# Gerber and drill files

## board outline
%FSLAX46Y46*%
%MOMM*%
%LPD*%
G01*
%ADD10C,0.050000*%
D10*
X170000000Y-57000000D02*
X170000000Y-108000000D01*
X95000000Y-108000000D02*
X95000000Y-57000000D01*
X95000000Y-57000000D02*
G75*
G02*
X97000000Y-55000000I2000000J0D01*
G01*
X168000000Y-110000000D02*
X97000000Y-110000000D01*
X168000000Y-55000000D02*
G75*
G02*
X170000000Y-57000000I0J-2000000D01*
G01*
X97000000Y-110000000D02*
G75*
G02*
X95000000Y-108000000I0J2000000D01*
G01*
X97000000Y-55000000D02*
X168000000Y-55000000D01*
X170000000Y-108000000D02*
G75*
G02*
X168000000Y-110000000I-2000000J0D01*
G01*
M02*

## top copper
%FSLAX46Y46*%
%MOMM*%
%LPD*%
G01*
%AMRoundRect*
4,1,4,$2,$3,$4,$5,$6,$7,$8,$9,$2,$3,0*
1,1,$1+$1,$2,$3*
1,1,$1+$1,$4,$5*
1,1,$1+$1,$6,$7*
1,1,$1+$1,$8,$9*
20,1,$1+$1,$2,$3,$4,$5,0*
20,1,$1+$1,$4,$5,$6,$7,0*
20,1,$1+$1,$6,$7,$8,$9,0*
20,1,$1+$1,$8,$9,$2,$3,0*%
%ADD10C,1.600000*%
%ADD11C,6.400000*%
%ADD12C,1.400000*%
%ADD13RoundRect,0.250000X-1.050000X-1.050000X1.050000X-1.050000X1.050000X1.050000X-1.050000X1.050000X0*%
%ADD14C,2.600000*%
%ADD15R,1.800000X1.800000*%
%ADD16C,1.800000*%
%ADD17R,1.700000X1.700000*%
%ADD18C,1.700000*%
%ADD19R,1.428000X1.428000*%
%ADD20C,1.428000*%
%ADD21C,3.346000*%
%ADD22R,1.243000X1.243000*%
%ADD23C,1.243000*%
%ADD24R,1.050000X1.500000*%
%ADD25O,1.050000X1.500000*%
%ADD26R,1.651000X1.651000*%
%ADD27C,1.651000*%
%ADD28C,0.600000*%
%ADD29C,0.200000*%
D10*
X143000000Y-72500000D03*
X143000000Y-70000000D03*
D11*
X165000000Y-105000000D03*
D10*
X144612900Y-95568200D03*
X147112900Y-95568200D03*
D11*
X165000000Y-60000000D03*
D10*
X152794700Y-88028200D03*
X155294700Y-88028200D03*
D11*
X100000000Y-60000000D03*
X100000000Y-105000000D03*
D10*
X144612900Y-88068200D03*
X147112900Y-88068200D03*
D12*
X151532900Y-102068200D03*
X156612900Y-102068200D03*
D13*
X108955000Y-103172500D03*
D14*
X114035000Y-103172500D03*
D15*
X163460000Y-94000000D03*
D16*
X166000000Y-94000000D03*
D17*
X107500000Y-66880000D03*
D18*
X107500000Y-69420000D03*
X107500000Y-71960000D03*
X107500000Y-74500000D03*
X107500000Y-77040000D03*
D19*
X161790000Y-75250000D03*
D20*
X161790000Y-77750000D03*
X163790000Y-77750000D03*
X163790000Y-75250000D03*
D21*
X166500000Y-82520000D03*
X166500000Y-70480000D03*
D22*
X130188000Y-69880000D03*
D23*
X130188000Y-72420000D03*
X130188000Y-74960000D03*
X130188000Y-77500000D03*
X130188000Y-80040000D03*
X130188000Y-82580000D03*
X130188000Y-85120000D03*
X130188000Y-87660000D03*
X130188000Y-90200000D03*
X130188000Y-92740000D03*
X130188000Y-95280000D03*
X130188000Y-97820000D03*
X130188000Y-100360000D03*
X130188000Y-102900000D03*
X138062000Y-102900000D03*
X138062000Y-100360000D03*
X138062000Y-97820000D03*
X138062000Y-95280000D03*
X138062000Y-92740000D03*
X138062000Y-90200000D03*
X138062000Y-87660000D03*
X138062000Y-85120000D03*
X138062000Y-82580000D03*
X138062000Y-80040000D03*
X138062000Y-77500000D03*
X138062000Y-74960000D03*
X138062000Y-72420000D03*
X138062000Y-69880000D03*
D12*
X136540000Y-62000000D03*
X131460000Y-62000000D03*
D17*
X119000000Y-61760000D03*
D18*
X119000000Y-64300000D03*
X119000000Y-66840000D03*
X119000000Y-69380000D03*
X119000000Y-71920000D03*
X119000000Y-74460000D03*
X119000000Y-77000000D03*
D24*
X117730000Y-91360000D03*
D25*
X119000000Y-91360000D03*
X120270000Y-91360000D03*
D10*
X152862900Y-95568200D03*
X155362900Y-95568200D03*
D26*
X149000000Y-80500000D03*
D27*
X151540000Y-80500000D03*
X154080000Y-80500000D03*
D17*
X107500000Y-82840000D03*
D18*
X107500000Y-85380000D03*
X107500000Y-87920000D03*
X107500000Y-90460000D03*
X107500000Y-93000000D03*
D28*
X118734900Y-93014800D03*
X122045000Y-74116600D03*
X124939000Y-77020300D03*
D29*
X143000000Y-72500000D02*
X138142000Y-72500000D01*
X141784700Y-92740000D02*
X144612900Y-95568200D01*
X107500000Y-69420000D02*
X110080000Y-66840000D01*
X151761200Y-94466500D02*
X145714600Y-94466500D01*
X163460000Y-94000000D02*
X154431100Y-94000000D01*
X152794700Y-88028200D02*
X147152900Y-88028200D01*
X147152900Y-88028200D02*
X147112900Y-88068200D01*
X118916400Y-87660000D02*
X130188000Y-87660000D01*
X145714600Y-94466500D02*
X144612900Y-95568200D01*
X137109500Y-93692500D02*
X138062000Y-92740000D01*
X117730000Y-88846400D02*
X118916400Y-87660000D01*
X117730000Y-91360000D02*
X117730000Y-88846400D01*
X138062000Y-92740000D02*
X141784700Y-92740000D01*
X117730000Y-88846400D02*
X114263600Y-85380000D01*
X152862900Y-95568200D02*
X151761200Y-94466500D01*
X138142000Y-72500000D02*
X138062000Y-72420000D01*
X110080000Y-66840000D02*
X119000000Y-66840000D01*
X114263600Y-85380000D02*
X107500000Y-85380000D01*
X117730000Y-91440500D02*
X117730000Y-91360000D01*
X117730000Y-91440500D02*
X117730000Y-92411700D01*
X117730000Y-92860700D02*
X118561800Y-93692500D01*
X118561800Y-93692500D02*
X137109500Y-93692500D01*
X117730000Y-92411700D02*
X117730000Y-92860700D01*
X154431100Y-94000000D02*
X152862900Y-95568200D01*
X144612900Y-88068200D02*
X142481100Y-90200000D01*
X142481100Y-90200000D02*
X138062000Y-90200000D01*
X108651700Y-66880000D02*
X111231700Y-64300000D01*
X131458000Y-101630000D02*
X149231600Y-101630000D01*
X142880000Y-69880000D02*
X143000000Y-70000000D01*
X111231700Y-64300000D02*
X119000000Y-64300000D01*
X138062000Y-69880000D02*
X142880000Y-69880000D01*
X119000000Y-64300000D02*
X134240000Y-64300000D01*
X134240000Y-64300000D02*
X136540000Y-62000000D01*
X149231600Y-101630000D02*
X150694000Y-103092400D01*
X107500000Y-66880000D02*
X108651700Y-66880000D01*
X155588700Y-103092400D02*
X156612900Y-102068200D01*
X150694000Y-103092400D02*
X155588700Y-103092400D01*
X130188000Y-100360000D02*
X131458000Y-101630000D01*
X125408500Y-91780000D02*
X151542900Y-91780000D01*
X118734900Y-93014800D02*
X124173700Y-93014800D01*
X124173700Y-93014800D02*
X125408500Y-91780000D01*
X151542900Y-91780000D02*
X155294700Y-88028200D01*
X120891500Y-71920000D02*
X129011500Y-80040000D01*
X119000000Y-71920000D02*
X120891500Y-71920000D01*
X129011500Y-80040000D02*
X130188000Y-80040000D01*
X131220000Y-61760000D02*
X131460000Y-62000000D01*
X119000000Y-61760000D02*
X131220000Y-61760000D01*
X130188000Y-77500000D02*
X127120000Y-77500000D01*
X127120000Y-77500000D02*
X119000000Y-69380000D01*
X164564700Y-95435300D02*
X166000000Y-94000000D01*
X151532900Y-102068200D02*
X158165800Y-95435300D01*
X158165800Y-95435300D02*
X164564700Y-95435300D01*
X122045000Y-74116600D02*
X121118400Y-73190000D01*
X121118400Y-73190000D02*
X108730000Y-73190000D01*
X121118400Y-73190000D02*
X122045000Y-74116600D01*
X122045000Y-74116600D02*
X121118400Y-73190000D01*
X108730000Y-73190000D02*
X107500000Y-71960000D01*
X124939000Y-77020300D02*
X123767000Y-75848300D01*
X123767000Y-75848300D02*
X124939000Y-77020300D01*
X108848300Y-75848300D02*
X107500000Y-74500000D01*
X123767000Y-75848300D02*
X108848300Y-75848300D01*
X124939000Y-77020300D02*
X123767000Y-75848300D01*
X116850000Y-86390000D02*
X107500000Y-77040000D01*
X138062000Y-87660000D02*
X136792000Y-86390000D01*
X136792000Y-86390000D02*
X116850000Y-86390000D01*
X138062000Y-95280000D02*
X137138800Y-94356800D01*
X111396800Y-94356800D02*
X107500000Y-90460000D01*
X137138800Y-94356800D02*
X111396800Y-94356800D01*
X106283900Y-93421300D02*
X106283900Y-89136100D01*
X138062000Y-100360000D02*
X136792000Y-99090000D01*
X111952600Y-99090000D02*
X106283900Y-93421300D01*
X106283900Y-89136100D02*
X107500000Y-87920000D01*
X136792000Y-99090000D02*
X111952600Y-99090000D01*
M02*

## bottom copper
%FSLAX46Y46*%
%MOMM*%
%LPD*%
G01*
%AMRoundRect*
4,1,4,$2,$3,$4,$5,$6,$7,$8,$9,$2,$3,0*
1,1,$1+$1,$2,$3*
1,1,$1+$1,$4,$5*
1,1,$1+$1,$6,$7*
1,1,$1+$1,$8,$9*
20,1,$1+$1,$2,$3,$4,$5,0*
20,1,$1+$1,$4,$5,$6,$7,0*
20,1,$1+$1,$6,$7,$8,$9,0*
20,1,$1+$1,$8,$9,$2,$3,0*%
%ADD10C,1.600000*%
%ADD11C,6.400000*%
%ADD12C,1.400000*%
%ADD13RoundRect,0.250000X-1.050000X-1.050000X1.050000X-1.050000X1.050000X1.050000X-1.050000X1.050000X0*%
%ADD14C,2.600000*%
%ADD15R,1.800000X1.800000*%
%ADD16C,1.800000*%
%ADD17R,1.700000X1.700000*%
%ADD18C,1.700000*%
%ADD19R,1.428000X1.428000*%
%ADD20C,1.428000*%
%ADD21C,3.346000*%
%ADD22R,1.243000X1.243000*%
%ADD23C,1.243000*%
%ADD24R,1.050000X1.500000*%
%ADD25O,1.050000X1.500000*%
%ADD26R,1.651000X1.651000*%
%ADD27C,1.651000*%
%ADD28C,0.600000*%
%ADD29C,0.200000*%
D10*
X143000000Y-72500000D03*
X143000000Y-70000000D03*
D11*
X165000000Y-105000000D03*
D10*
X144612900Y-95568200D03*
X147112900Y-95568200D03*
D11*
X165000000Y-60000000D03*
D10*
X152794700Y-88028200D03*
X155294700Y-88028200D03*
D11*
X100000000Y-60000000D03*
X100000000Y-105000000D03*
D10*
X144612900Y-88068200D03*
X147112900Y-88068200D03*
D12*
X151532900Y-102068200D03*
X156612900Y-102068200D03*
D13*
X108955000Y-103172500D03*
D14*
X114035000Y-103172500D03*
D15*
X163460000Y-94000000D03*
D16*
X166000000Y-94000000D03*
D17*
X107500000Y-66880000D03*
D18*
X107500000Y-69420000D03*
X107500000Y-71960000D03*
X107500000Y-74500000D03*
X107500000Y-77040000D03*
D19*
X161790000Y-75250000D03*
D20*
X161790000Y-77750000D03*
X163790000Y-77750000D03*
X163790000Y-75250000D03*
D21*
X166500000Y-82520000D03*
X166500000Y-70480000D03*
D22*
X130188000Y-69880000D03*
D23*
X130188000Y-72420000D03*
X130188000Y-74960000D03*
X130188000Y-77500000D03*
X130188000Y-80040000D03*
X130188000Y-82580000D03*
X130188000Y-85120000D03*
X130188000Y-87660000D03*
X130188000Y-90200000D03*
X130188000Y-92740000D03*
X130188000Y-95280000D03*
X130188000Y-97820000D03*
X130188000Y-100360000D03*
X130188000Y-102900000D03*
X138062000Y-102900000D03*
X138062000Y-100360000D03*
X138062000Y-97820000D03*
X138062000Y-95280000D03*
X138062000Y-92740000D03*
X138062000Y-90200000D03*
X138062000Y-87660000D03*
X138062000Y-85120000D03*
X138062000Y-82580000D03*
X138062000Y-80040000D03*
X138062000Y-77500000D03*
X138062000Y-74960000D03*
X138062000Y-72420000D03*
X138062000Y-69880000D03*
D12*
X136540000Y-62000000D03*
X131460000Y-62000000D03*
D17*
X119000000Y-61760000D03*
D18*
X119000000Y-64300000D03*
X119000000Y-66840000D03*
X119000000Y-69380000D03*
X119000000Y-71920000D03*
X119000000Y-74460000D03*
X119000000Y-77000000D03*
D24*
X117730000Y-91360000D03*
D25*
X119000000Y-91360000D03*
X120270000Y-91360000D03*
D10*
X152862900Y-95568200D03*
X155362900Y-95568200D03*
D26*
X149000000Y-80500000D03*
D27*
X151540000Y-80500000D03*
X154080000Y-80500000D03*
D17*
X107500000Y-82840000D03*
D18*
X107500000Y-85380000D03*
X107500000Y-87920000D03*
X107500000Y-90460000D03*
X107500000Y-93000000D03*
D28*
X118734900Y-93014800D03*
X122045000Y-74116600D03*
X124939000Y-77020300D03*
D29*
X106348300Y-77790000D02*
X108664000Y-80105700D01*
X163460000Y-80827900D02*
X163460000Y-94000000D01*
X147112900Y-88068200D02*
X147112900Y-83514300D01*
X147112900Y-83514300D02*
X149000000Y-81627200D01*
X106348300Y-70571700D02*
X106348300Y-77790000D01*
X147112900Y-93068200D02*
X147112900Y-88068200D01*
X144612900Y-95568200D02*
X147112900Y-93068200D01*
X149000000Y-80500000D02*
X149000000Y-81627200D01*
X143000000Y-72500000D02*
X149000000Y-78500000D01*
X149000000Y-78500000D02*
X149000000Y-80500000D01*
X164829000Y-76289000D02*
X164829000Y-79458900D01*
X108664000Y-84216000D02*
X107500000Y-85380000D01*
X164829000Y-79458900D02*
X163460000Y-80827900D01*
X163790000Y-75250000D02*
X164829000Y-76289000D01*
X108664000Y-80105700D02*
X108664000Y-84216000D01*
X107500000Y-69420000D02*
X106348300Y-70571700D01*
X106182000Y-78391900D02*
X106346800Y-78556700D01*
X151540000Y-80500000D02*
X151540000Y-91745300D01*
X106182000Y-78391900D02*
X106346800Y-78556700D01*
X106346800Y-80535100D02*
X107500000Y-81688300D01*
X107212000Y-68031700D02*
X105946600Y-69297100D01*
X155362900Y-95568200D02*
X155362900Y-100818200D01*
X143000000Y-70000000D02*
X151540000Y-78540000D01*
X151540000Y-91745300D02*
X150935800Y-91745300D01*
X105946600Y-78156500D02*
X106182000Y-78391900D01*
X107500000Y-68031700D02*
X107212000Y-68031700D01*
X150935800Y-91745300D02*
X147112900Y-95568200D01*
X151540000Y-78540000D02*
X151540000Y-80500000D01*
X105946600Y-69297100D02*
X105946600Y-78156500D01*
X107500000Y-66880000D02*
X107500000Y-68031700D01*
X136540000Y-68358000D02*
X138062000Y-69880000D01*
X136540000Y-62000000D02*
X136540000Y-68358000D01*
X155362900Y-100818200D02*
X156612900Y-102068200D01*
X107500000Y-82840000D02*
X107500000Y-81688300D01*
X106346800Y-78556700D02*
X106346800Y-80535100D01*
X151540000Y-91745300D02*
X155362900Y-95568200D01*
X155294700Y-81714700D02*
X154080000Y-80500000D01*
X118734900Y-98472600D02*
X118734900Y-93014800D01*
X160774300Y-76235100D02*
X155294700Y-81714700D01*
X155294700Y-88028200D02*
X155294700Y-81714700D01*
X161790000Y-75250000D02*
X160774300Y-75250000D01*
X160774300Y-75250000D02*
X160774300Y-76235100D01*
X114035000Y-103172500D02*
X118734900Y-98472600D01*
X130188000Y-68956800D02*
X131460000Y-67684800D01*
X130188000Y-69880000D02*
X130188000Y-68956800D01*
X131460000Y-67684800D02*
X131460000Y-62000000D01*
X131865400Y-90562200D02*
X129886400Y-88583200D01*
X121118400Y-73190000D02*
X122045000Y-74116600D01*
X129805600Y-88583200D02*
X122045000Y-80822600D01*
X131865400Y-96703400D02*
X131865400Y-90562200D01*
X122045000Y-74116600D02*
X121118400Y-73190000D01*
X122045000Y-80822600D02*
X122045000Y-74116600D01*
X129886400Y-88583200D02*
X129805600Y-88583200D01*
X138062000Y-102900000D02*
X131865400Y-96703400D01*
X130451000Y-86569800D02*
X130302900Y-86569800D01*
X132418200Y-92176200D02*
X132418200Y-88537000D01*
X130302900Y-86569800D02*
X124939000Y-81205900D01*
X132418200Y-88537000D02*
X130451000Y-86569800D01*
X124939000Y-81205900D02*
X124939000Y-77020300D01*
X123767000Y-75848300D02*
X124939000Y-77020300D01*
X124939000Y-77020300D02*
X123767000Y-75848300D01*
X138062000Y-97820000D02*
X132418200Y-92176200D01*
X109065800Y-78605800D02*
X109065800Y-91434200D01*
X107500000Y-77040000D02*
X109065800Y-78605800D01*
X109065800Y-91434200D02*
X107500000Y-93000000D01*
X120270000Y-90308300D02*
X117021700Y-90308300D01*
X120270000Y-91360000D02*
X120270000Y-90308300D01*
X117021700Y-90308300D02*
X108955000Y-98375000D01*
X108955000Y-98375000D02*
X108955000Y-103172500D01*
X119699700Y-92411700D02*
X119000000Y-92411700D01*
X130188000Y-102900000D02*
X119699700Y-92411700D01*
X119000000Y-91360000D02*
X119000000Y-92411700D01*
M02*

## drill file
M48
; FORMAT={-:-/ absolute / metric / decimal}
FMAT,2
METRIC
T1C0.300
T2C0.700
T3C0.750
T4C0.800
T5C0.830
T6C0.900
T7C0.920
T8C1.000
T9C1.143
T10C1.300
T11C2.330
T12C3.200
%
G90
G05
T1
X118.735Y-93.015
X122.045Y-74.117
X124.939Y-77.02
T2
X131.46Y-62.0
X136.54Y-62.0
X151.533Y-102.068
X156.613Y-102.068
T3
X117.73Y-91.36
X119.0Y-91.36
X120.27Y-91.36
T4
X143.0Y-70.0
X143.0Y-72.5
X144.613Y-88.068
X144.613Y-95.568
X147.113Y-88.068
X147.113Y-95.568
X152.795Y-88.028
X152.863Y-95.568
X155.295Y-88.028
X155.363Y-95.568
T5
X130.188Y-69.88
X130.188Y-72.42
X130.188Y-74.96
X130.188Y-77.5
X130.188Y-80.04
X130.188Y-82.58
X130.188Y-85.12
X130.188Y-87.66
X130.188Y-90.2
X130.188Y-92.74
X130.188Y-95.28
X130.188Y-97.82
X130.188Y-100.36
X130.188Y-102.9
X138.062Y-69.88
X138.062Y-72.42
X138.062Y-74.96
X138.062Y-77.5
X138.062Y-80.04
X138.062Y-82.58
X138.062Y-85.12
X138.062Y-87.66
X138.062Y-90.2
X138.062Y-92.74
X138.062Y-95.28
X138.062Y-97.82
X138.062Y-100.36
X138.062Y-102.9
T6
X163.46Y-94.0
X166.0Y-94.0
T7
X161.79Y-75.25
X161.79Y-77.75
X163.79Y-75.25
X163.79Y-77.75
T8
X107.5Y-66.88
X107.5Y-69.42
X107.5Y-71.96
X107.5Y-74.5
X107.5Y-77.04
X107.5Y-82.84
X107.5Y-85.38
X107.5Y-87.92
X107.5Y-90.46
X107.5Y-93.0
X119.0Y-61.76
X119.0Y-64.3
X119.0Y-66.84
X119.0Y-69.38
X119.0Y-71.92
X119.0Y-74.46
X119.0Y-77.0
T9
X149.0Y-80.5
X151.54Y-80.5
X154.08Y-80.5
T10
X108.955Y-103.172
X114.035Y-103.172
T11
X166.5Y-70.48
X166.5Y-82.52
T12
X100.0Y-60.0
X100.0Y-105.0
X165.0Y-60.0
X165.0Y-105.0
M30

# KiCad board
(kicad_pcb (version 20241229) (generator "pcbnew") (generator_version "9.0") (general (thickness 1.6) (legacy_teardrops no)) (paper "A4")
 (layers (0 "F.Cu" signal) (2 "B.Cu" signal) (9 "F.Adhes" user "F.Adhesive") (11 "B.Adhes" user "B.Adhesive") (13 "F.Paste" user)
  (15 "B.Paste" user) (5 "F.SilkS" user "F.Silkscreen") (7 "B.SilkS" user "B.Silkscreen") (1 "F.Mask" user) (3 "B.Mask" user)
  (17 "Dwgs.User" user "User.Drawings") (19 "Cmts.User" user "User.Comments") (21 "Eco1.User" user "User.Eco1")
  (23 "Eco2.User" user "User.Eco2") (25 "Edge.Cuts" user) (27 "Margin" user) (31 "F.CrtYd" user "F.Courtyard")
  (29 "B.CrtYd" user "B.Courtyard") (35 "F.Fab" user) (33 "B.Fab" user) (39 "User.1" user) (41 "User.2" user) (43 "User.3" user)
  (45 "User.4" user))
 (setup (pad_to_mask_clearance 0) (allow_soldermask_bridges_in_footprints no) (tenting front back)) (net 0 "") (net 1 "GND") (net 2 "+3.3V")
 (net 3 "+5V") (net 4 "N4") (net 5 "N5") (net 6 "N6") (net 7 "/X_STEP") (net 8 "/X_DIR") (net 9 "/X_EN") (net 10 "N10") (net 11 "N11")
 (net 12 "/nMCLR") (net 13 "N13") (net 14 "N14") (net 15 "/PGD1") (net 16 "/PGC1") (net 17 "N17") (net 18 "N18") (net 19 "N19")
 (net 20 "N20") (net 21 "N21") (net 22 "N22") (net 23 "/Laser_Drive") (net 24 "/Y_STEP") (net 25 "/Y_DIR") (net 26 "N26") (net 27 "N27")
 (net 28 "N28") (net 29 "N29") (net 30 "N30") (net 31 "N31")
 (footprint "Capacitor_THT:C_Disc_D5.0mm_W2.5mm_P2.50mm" (layer "F.Cu") (at 143 72.5 90)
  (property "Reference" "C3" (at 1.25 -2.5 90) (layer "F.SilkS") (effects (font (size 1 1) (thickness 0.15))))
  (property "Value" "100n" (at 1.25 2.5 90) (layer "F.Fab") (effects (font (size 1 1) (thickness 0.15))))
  (pad "1" thru_hole circle (at 0 0 90) (size 1.6 1.6) (drill 0.8) (layers "*.Cu" "*.Mask") (remove_unused_layers no) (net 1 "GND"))
  (pad "2" thru_hole circle (at 2.5 0 90) (size 1.6 1.6) (drill 0.8) (layers "*.Cu" "*.Mask") (remove_unused_layers no) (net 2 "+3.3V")))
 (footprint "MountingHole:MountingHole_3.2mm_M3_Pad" (layer "F.Cu") (at 165 105)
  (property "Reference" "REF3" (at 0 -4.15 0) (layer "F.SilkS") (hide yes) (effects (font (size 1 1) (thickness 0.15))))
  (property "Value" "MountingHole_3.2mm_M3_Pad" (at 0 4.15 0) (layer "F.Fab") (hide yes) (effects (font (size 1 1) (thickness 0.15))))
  (pad "1" thru_hole circle (at 0 0) (size 6.4 6.4) (drill 3.2) (layers "*.Cu" "*.Mask") (remove_unused_layers no) (zone_connect 2)))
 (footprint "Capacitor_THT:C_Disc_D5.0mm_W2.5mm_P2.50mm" (layer "F.Cu") (at 144.6129 95.5682)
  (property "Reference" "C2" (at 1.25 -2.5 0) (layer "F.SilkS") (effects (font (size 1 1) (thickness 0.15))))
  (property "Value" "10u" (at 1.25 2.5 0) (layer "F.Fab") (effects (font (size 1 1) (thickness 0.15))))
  (pad "1" thru_hole circle (at 0 0) (size 1.6 1.6) (drill 0.8) (layers "*.Cu" "*.Mask") (remove_unused_layers no) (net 1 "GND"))
  (pad "2" thru_hole circle (at 2.5 0) (size 1.6 1.6) (drill 0.8) (layers "*.Cu" "*.Mask") (remove_unused_layers no) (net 2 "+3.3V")))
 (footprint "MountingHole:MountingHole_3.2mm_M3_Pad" (layer "F.Cu") (at 165 60)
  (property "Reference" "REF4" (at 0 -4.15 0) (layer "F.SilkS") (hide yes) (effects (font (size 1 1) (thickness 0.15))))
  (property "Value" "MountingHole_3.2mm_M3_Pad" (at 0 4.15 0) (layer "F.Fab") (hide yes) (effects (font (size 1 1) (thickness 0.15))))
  (pad "1" thru_hole circle (at 0 0) (size 6.4 6.4) (drill 3.2) (layers "*.Cu" "*.Mask") (remove_unused_layers no) (zone_connect 2)))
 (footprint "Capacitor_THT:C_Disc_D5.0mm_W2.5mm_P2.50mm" (layer "F.Cu") (at 152.7947 88.0282)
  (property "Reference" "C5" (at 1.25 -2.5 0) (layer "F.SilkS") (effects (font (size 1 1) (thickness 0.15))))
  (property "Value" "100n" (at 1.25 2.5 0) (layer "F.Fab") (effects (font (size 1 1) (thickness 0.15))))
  (pad "1" thru_hole circle (at 0 0) (size 1.6 1.6) (drill 0.8) (layers "*.Cu" "*.Mask") (remove_unused_layers no) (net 1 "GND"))
  (pad "2" thru_hole circle (at 2.5 0) (size 1.6 1.6) (drill 0.8) (layers "*.Cu" "*.Mask") (remove_unused_layers no) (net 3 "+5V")))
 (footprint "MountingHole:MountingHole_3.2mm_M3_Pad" (layer "F.Cu") (at 100 60)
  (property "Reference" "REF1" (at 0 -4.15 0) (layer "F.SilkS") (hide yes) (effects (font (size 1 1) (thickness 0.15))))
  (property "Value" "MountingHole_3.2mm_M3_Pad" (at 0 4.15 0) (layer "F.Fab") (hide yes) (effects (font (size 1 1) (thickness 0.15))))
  (pad "1" thru_hole circle (at 0 0) (size 6.4 6.4) (drill 3.2) (layers "*.Cu" "*.Mask") (remove_unused_layers no) (zone_connect 2)))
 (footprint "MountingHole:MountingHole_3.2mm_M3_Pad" (layer "F.Cu") (at 100 105)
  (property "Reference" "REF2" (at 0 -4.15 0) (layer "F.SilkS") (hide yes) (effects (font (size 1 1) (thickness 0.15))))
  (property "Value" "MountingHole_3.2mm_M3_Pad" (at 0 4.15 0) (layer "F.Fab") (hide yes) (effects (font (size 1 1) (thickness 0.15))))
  (pad "1" thru_hole circle (at 0 0) (size 6.4 6.4) (drill 3.2) (layers "*.Cu" "*.Mask") (remove_unused_layers no) (zone_connect 2)))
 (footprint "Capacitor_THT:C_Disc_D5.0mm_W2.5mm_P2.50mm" (layer "F.Cu") (at 144.6129 88.0682)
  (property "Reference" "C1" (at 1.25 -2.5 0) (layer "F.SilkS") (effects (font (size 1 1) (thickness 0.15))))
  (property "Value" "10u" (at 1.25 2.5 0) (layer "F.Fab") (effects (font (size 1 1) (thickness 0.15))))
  (pad "1" thru_hole circle (at 0 0) (size 1.6 1.6) (drill 0.8) (layers "*.Cu" "*.Mask") (remove_unused_layers no) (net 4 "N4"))
  (pad "2" thru_hole circle (at 2.5 0) (size 1.6 1.6) (drill 0.8) (layers "*.Cu" "*.Mask") (remove_unused_layers no) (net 1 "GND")))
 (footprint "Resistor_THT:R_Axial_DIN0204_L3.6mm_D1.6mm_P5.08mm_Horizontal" (layer "F.Cu") (at 151.5329 102.0682)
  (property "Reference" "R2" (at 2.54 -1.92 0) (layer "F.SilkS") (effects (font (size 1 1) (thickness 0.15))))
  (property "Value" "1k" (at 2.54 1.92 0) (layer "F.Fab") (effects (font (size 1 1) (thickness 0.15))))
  (pad "1" thru_hole circle (at 0 0) (size 1.4 1.4) (drill 0.7) (layers "*.Cu" "*.Mask") (remove_unused_layers no) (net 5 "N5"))
  (pad "2" thru_hole circle (at 5.08 0) (size 1.4 1.4) (drill 0.7) (layers "*.Cu" "*.Mask") (remove_unused_layers no) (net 2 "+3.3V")))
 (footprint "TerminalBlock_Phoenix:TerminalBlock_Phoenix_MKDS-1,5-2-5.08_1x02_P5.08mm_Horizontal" (layer "F.Cu") (at 108.955 103.1725)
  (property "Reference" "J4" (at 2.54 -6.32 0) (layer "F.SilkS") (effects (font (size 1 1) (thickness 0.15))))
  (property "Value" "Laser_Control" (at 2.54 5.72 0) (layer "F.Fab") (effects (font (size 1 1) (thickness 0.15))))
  (pad "1" thru_hole roundrect (at 0 0) (size 2.6 2.6) (drill 1.3) (layers "*.Cu" "*.Mask") (remove_unused_layers no)
   (roundrect_rratio 0.096154) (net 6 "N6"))
  (pad "2" thru_hole circle (at 5.08 0) (size 2.6 2.6) (drill 1.3) (layers "*.Cu" "*.Mask") (remove_unused_layers no) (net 3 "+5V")))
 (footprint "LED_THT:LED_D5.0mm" (layer "F.Cu") (at 163.46 94)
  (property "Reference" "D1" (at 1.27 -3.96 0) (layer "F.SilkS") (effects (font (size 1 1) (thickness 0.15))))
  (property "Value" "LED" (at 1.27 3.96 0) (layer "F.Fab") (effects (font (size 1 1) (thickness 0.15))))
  (pad "1" thru_hole rect (at 0 0) (size 1.8 1.8) (drill 0.9) (layers "*.Cu" "*.Mask") (remove_unused_layers no) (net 1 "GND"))
  (pad "2" thru_hole circle (at 2.54 0) (size 1.8 1.8) (drill 0.9) (layers "*.Cu" "*.Mask") (remove_unused_layers no) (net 5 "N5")))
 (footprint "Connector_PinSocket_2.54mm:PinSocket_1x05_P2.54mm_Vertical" (layer "F.Cu") (at 107.5 66.88)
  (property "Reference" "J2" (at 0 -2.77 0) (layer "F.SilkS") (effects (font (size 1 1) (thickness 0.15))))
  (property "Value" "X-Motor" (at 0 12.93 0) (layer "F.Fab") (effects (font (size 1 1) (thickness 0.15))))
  (pad "1" thru_hole rect (at 0 0) (size 1.7 1.7) (drill 1) (layers "*.Cu" "*.Mask") (remove_unused_layers no) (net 2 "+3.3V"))
  (pad "2" thru_hole circle (at 0 2.54) (size 1.7 1.7) (drill 1) (layers "*.Cu" "*.Mask") (remove_unused_layers no) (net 1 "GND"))
  (pad "3" thru_hole circle (at 0 5.08) (size 1.7 1.7) (drill 1) (layers "*.Cu" "*.Mask") (remove_unused_layers no) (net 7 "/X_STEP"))
  (pad "4" thru_hole circle (at 0 7.62) (size 1.7 1.7) (drill 1) (layers "*.Cu" "*.Mask") (remove_unused_layers no) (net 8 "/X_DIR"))
  (pad "5" thru_hole circle (at 0 10.16) (size 1.7 1.7) (drill 1) (layers "*.Cu" "*.Mask") (remove_unused_layers no) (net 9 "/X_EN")))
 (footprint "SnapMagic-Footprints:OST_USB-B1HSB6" (layer "F.Cu") (at 166.5 76.5 90)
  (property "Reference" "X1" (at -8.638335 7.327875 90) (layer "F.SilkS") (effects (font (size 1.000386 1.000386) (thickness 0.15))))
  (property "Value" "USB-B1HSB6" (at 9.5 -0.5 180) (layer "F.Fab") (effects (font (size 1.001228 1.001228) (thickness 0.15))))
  (pad "1" thru_hole rect (at 1.25 -4.71 90) (size 1.428 1.428) (drill 0.92) (layers "*.Cu" "*.Mask") (remove_unused_layers no)
   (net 3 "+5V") (solder_mask_margin 0.102))
  (pad "2" thru_hole circle (at -1.25 -4.71 90) (size 1.428 1.428) (drill 0.92) (layers "*.Cu" "*.Mask") (remove_unused_layers no)
   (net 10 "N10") (solder_mask_margin 0.102))
  (pad "3" thru_hole circle (at -1.25 -2.71 90) (size 1.428 1.428) (drill 0.92) (layers "*.Cu" "*.Mask") (remove_unused_layers no)
   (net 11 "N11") (solder_mask_margin 0.102))
  (pad "4" thru_hole circle (at 1.25 -2.71 90) (size 1.428 1.428) (drill 0.92) (layers "*.Cu" "*.Mask") (remove_unused_layers no)
   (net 1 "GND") (solder_mask_margin 0.102))
  (pad "P1" thru_hole circle (at -6.02 0 90) (size 3.346 3.346) (drill 2.33) (layers "*.Cu" "*.Mask") (remove_unused_layers no)
   (solder_mask_margin 0.102))
  (pad "P2" thru_hole circle (at 6.02 0 90) (size 3.346 3.346) (drill 2.33) (layers "*.Cu" "*.Mask") (remove_unused_layers no)
   (solder_mask_margin 0.102)))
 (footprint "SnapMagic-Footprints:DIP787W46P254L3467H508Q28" (layer "F.Cu") (at 134.125 86.39)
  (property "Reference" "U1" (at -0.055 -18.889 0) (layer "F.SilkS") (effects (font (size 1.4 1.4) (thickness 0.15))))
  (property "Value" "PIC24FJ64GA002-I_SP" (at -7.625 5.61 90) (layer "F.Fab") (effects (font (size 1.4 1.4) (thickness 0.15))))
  (pad "1" thru_hole rect (at -3.937 -16.51) (size 1.243 1.243) (drill 0.83) (layers "*.Cu" "*.Mask") (remove_unused_layers no)
   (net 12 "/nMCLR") (solder_mask_margin 0.102))
  (pad "2" thru_hole circle (at -3.937 -13.97) (size 1.243 1.243) (drill 0.83) (layers "*.Cu" "*.Mask") (remove_unused_layers no)
   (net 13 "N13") (solder_mask_margin 0.102))
  (pad "3" thru_hole circle (at -3.937 -11.43) (size 1.243 1.243) (drill 0.83) (layers "*.Cu" "*.Mask") (remove_unused_layers no)
   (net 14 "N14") (solder_mask_margin 0.102))
  (pad "4" thru_hole circle (at -3.937 -8.89) (size 1.243 1.243) (drill 0.83) (layers "*.Cu" "*.Mask") (remove_unused_layers no)
   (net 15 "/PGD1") (solder_mask_margin 0.102))
  (pad "5" thru_hole circle (at -3.937 -6.35) (size 1.243 1.243) (drill 0.83) (layers "*.Cu" "*.Mask") (remove_unused_layers no)
   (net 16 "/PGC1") (solder_mask_margin 0.102))
  (pad "6" thru_hole circle (at -3.937 -3.81) (size 1.243 1.243) (drill 0.83) (layers "*.Cu" "*.Mask") (remove_unused_layers no)
   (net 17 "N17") (solder_mask_margin 0.102))
  (pad "7" thru_hole circle (at -3.937 -1.27) (size 1.243 1.243) (drill 0.83) (layers "*.Cu" "*.Mask") (remove_unused_layers no)
   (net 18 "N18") (solder_mask_margin 0.102))
  (pad "8" thru_hole circle (at -3.937 1.27) (size 1.243 1.243) (drill 0.83) (layers "*.Cu" "*.Mask") (remove_unused_layers no)
   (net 1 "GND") (solder_mask_margin 0.102))
  (pad "9" thru_hole circle (at -3.937 3.81) (size 1.243 1.243) (drill 0.83) (layers "*.Cu" "*.Mask") (remove_unused_layers no)
   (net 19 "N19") (solder_mask_margin 0.102))
  (pad "10" thru_hole circle (at -3.937 6.35) (size 1.243 1.243) (drill 0.83) (layers "*.Cu" "*.Mask") (remove_unused_layers no)
   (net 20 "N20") (solder_mask_margin 0.102))
  (pad "11" thru_hole circle (at -3.937 8.89) (size 1.243 1.243) (drill 0.83) (layers "*.Cu" "*.Mask") (remove_unused_layers no)
   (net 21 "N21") (solder_mask_margin 0.102))
  (pad "12" thru_hole circle (at -3.937 11.43) (size 1.243 1.243) (drill 0.83) (layers "*.Cu" "*.Mask") (remove_unused_layers no)
   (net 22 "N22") (solder_mask_margin 0.102))
  (pad "13" thru_hole circle (at -3.937 13.97) (size 1.243 1.243) (drill 0.83) (layers "*.Cu" "*.Mask") (remove_unused_layers no)
   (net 2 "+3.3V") (solder_mask_margin 0.102))
  (pad "14" thru_hole circle (at -3.937 16.51) (size 1.243 1.243) (drill 0.83) (layers "*.Cu" "*.Mask") (remove_unused_layers no)
   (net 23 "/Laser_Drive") (solder_mask_margin 0.102))
  (pad "15" thru_hole circle (at 3.937 16.51) (size 1.243 1.243) (drill 0.83) (layers "*.Cu" "*.Mask") (remove_unused_layers no)
   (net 7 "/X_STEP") (solder_mask_margin 0.102))
  (pad "16" thru_hole circle (at 3.937 13.97) (size 1.243 1.243) (drill 0.83) (layers "*.Cu" "*.Mask") (remove_unused_layers no)
   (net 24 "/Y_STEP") (solder_mask_margin 0.102))
  (pad "17" thru_hole circle (at 3.937 11.43) (size 1.243 1.243) (drill 0.83) (layers "*.Cu" "*.Mask") (remove_unused_layers no)
   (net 8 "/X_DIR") (solder_mask_margin 0.102))
  (pad "18" thru_hole circle (at 3.937 8.89) (size 1.243 1.243) (drill 0.83) (layers "*.Cu" "*.Mask") (remove_unused_layers no)
   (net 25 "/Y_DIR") (solder_mask_margin 0.102))
  (pad "19" thru_hole circle (at 3.937 6.35) (size 1.243 1.243) (drill 0.83) (layers "*.Cu" "*.Mask") (remove_unused_layers no)
   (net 1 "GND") (solder_mask_margin 0.102))
  (pad "20" thru_hole circle (at 3.937 3.81) (size 1.243 1.243) (drill 0.83) (layers "*.Cu" "*.Mask") (remove_unused_layers no) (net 4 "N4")
   (solder_mask_margin 0.102))
  (pad "21" thru_hole circle (at 3.937 1.27) (size 1.243 1.243) (drill 0.83) (layers "*.Cu" "*.Mask") (remove_unused_layers no)
   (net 9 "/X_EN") (solder_mask_margin 0.102))
  (pad "22" thru_hole circle (at 3.937 -1.27) (size 1.243 1.243) (drill 0.83) (layers "*.Cu" "*.Mask") (remove_unused_layers no)
   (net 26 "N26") (solder_mask_margin 0.102))
  (pad "23" thru_hole circle (at 3.937 -3.81) (size 1.243 1.243) (drill 0.83) (layers "*.Cu" "*.Mask") (remove_unused_layers no)
   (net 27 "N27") (solder_mask_margin 0.102))
  (pad "24" thru_hole circle (at 3.937 -6.35) (size 1.243 1.243) (drill 0.83) (layers "*.Cu" "*.Mask") (remove_unused_layers no)
   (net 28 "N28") (solder_mask_margin 0.102))
  (pad "25" thru_hole circle (at 3.937 -8.89) (size 1.243 1.243) (drill 0.83) (layers "*.Cu" "*.Mask") (remove_unused_layers no)
   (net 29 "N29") (solder_mask_margin 0.102))
  (pad "26" thru_hole circle (at 3.937 -11.43) (size 1.243 1.243) (drill 0.83) (layers "*.Cu" "*.Mask") (remove_unused_layers no)
   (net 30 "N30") (solder_mask_margin 0.102))
  (pad "27" thru_hole circle (at 3.937 -13.97) (size 1.243 1.243) (drill 0.83) (layers "*.Cu" "*.Mask") (remove_unused_layers no)
   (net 1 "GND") (solder_mask_margin 0.102))
  (pad "28" thru_hole circle (at 3.937 -16.51) (size 1.243 1.243) (drill 0.83) (layers "*.Cu" "*.Mask") (remove_unused_layers no)
   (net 2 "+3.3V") (solder_mask_margin 0.102)))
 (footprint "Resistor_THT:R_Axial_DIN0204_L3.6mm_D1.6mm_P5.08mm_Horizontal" (layer "F.Cu") (at 136.54 62 180)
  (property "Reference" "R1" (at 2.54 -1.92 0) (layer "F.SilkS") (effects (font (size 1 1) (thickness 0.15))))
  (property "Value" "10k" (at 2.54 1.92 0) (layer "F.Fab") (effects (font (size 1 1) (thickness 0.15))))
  (pad "1" thru_hole circle (at 0 0 180) (size 1.4 1.4) (drill 0.7) (layers "*.Cu" "*.Mask") (remove_unused_layers no) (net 2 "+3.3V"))
  (pad "2" thru_hole circle (at 5.08 0 180) (size 1.4 1.4) (drill 0.7) (layers "*.Cu" "*.Mask") (remove_unused_layers no) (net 12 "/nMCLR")))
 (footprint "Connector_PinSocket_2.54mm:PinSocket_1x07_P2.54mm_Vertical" (layer "F.Cu") (at 119 61.76)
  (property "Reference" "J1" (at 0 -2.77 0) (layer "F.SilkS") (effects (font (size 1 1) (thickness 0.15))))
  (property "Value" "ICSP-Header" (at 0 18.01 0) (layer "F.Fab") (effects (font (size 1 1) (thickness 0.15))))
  (pad "1" thru_hole rect (at 0 0) (size 1.7 1.7) (drill 1) (layers "*.Cu" "*.Mask") (remove_unused_layers no) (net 12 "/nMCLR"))
  (pad "2" thru_hole circle (at 0 2.54) (size 1.7 1.7) (drill 1) (layers "*.Cu" "*.Mask") (remove_unused_layers no) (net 2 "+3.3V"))
  (pad "3" thru_hole circle (at 0 5.08) (size 1.7 1.7) (drill 1) (layers "*.Cu" "*.Mask") (remove_unused_layers no) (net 1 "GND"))
  (pad "4" thru_hole circle (at 0 7.62) (size 1.7 1.7) (drill 1) (layers "*.Cu" "*.Mask") (remove_unused_layers no) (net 15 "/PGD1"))
  (pad "5" thru_hole circle (at 0 10.16) (size 1.7 1.7) (drill 1) (layers "*.Cu" "*.Mask") (remove_unused_layers no) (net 16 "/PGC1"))
  (pad "6" thru_hole circle (at 0 12.7) (size 1.7 1.7) (drill 1) (layers "*.Cu" "*.Mask") (remove_unused_layers no) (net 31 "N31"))
  (pad "7" thru_hole circle (at 0 15.24) (size 1.7 1.7) (drill 1) (layers "*.Cu" "*.Mask") (remove_unused_layers no)))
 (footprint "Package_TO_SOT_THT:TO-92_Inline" (layer "F.Cu") (at 117.73 91.36)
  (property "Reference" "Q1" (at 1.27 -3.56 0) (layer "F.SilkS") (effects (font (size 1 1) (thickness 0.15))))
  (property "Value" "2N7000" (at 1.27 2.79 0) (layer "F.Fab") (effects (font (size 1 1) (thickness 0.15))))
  (pad "1" thru_hole rect (at 0 0) (size 1.05 1.5) (drill 0.75) (layers "*.Cu" "*.Mask") (remove_unused_layers no) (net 1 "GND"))
  (pad "2" thru_hole oval (at 1.27 0) (size 1.05 1.5) (drill 0.75) (layers "*.Cu" "*.Mask") (remove_unused_layers no)
   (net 23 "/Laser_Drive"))
  (pad "3" thru_hole oval (at 2.54 0) (size 1.05 1.5) (drill 0.75) (layers "*.Cu" "*.Mask") (remove_unused_layers no) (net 6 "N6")))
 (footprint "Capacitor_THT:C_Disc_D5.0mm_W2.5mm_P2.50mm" (layer "F.Cu") (at 152.8629 95.5682)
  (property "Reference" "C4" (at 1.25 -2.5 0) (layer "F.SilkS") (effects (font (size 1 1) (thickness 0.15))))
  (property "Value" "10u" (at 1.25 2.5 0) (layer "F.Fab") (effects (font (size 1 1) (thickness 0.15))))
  (pad "1" thru_hole circle (at 0 0) (size 1.6 1.6) (drill 0.8) (layers "*.Cu" "*.Mask") (remove_unused_layers no) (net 1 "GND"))
  (pad "2" thru_hole circle (at 2.5 0) (size 1.6 1.6) (drill 0.8) (layers "*.Cu" "*.Mask") (remove_unused_layers no) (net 2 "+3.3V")))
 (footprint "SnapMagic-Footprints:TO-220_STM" (layer "F.Cu") (at 149 80.5)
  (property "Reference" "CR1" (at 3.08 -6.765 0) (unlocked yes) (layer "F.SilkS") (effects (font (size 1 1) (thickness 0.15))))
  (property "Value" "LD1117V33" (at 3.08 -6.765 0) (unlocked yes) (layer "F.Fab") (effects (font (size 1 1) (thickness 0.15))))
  (pad "1" thru_hole rect (at 0 0) (size 1.651 1.651) (drill 1.143) (layers "*.Cu" "*.Mask") (remove_unused_layers no) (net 1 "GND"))
  (pad "2" thru_hole circle (at 2.54 0) (size 1.651 1.651) (drill 1.143) (layers "*.Cu" "*.Mask") (remove_unused_layers no) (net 2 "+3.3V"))
  (pad "3" thru_hole circle (at 5.08 0) (size 1.651 1.651) (drill 1.143) (layers "*.Cu" "*.Mask") (remove_unused_layers no) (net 3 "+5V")))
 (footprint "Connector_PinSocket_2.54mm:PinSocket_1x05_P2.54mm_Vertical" (layer "F.Cu") (at 107.5 82.84)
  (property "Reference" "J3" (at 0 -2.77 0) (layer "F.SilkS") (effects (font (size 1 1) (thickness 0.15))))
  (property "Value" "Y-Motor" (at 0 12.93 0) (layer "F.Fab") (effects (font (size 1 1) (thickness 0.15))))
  (pad "1" thru_hole rect (at 0 0) (size 1.7 1.7) (drill 1) (layers "*.Cu" "*.Mask") (remove_unused_layers no) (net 2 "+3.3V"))
  (pad "2" thru_hole circle (at 0 2.54) (size 1.7 1.7) (drill 1) (layers "*.Cu" "*.Mask") (remove_unused_layers no) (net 1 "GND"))
  (pad "3" thru_hole circle (at 0 5.08) (size 1.7 1.7) (drill 1) (layers "*.Cu" "*.Mask") (remove_unused_layers no) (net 24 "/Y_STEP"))
  (pad "4" thru_hole circle (at 0 7.62) (size 1.7 1.7) (drill 1) (layers "*.Cu" "*.Mask") (remove_unused_layers no) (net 25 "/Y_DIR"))
  (pad "5" thru_hole circle (at 0 10.16) (size 1.7 1.7) (drill 1) (layers "*.Cu" "*.Mask") (remove_unused_layers no) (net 9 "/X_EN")))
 (gr_line (start 170 57) (end 170 108) (stroke (width 0.05) (type default)) (layer "Edge.Cuts"))
 (gr_line (start 95 108) (end 95 57) (stroke (width 0.05) (type default)) (layer "Edge.Cuts"))
 (gr_arc (start 95 57) (mid 95.585786 55.585786) (end 97 55) (stroke (width 0.05) (type default)) (layer "Edge.Cuts"))
 (gr_line (start 168 110) (end 97 110) (stroke (width 0.05) (type default)) (layer "Edge.Cuts"))
 (gr_arc (start 168 55) (mid 169.414214 55.585786) (end 170 57) (stroke (width 0.05) (type default)) (layer "Edge.Cuts"))
 (gr_arc (start 97 110) (mid 95.585786 109.414214) (end 95 108) (stroke (width 0.05) (type default)) (layer "Edge.Cuts"))
 (gr_line (start 97 55) (end 168 55) (stroke (width 0.05) (type default)) (layer "Edge.Cuts"))
 (gr_arc (start 170 108) (mid 169.414214 109.414214) (end 168 110) (stroke (width 0.05) (type default)) (layer "Edge.Cuts"))
 (segment (start 143 72.5) (end 138.142 72.5) (width 0.2) (layer "F.Cu") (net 1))
 (segment (start 141.7847 92.74) (end 144.6129 95.5682) (width 0.2) (layer "F.Cu") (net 1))
 (segment (start 107.5 69.42) (end 110.08 66.84) (width 0.2) (layer "F.Cu") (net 1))
 (segment (start 151.7612 94.4665) (end 145.7146 94.4665) (width 0.2) (layer "F.Cu") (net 1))
 (segment (start 163.46 94) (end 154.4311 94) (width 0.2) (layer "F.Cu") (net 1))
 (segment (start 152.7947 88.0282) (end 147.1529 88.0282) (width 0.2) (layer "F.Cu") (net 1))
 (segment (start 147.1529 88.0282) (end 147.1129 88.0682) (width 0.2) (layer "F.Cu") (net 1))
 (segment (start 118.9164 87.66) (end 130.188 87.66) (width 0.2) (layer "F.Cu") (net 1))
 (segment (start 145.7146 94.4665) (end 144.6129 95.5682) (width 0.2) (layer "F.Cu") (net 1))
 (segment (start 137.1095 93.6925) (end 138.062 92.74) (width 0.2) (layer "F.Cu") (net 1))
 (segment (start 117.73 88.8464) (end 118.9164 87.66) (width 0.2) (layer "F.Cu") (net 1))
 (segment (start 117.73 91.36) (end 117.73 88.8464) (width 0.2) (layer "F.Cu") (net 1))
 (segment (start 138.062 92.74) (end 141.7847 92.74) (width 0.2) (layer "F.Cu") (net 1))
 (segment (start 117.73 88.8464) (end 114.2636 85.38) (width 0.2) (layer "F.Cu") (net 1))
 (segment (start 152.8629 95.5682) (end 151.7612 94.4665) (width 0.2) (layer "F.Cu") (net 1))
 (segment (start 138.142 72.5) (end 138.062 72.42) (width 0.2) (layer "F.Cu") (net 1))
 (segment (start 110.08 66.84) (end 119 66.84) (width 0.2) (layer "F.Cu") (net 1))
 (segment (start 114.2636 85.38) (end 107.5 85.38) (width 0.2) (layer "F.Cu") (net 1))
 (segment (start 117.73 91.4405) (end 117.73 91.36) (width 0.2) (layer "F.Cu") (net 1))
 (segment (start 117.73 91.4405) (end 117.73 92.4117) (width 0.2) (layer "F.Cu") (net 1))
 (segment (start 117.73 92.8607) (end 118.5618 93.6925) (width 0.2) (layer "F.Cu") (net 1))
 (segment (start 118.5618 93.6925) (end 137.1095 93.6925) (width 0.2) (layer "F.Cu") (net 1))
 (segment (start 117.73 92.4117) (end 117.73 92.8607) (width 0.2) (layer "F.Cu") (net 1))
 (segment (start 154.4311 94) (end 152.8629 95.5682) (width 0.2) (layer "F.Cu") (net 1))
 (segment (start 106.3483 77.79) (end 108.664 80.1057) (width 0.2) (layer "B.Cu") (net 1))
 (segment (start 163.46 80.8279) (end 163.46 94) (width 0.2) (layer "B.Cu") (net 1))
 (segment (start 147.1129 88.0682) (end 147.1129 83.5143) (width 0.2) (layer "B.Cu") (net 1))
 (segment (start 147.1129 83.5143) (end 149 81.6272) (width 0.2) (layer "B.Cu") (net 1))
 (segment (start 106.3483 70.5717) (end 106.3483 77.79) (width 0.2) (layer "B.Cu") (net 1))
 (segment (start 147.1129 93.0682) (end 147.1129 88.0682) (width 0.2) (layer "B.Cu") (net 1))
 (segment (start 144.6129 95.5682) (end 147.1129 93.0682) (width 0.2) (layer "B.Cu") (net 1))
 (segment (start 149 80.5) (end 149 81.6272) (width 0.2) (layer "B.Cu") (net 1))
 (segment (start 143 72.5) (end 149 78.5) (width 0.2) (layer "B.Cu") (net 1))
 (segment (start 149 78.5) (end 149 80.5) (width 0.2) (layer "B.Cu") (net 1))
 (segment (start 164.829 76.289) (end 164.829 79.4589) (width 0.2) (layer "B.Cu") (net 1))
 (segment (start 108.664 84.216) (end 107.5 85.38) (width 0.2) (layer "B.Cu") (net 1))
 (segment (start 164.829 79.4589) (end 163.46 80.8279) (width 0.2) (layer "B.Cu") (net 1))
 (segment (start 163.79 75.25) (end 164.829 76.289) (width 0.2) (layer "B.Cu") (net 1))
 (segment (start 108.664 80.1057) (end 108.664 84.216) (width 0.2) (layer "B.Cu") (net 1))
 (segment (start 107.5 69.42) (end 106.3483 70.5717) (width 0.2) (layer "B.Cu") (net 1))
 (segment (start 144.6129 88.0682) (end 142.4811 90.2) (width 0.2) (layer "F.Cu") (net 4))
 (segment (start 142.4811 90.2) (end 138.062 90.2) (width 0.2) (layer "F.Cu") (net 4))
 (segment (start 108.6517 66.88) (end 111.2317 64.3) (width 0.2) (layer "F.Cu") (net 2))
 (segment (start 131.458 101.63) (end 149.2316 101.63) (width 0.2) (layer "F.Cu") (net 2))
 (segment (start 142.88 69.88) (end 143 70) (width 0.2) (layer "F.Cu") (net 2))
 (segment (start 111.2317 64.3) (end 119 64.3) (width 0.2) (layer "F.Cu") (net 2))
 (segment (start 138.062 69.88) (end 142.88 69.88) (width 0.2) (layer "F.Cu") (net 2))
 (segment (start 119 64.3) (end 134.24 64.3) (width 0.2) (layer "F.Cu") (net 2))
 (segment (start 134.24 64.3) (end 136.54 62) (width 0.2) (layer "F.Cu") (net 2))
 (segment (start 149.2316 101.63) (end 150.694 103.0924) (width 0.2) (layer "F.Cu") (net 2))
 (segment (start 107.5 66.88) (end 108.6517 66.88) (width 0.2) (layer "F.Cu") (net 2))
 (segment (start 155.5887 103.0924) (end 156.6129 102.0682) (width 0.2) (layer "F.Cu") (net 2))
 (segment (start 150.694 103.0924) (end 155.5887 103.0924) (width 0.2) (layer "F.Cu") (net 2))
 (segment (start 130.188 100.36) (end 131.458 101.63) (width 0.2) (layer "F.Cu") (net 2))
 (segment (start 106.182 78.3919) (end 106.3468 78.5567) (width 0.2) (layer "B.Cu") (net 2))
 (segment (start 151.54 80.5) (end 151.54 91.7453) (width 0.2) (layer "B.Cu") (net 2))
 (segment (start 106.182 78.3919) (end 106.3468 78.5567) (width 0.2) (layer "B.Cu") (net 2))
 (segment (start 106.3468 80.5351) (end 107.5 81.6883) (width 0.2) (layer "B.Cu") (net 2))
 (segment (start 107.212 68.0317) (end 105.9466 69.2971) (width 0.2) (layer "B.Cu") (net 2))
 (segment (start 155.3629 95.5682) (end 155.3629 100.8182) (width 0.2) (layer "B.Cu") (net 2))
 (segment (start 143 70) (end 151.54 78.54) (width 0.2) (layer "B.Cu") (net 2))
 (segment (start 151.54 91.7453) (end 150.9358 91.7453) (width 0.2) (layer "B.Cu") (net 2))
 (segment (start 105.9466 78.1565) (end 106.182 78.3919) (width 0.2) (layer "B.Cu") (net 2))
 (segment (start 107.5 68.0317) (end 107.212 68.0317) (width 0.2) (layer "B.Cu") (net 2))
 (segment (start 150.9358 91.7453) (end 147.1129 95.5682) (width 0.2) (layer "B.Cu") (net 2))
 (segment (start 151.54 78.54) (end 151.54 80.5) (width 0.2) (layer "B.Cu") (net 2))
 (segment (start 105.9466 69.2971) (end 105.9466 78.1565) (width 0.2) (layer "B.Cu") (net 2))
 (segment (start 107.5 66.88) (end 107.5 68.0317) (width 0.2) (layer "B.Cu") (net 2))
 (segment (start 136.54 68.358) (end 138.062 69.88) (width 0.2) (layer "B.Cu") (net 2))
 (segment (start 136.54 62) (end 136.54 68.358) (width 0.2) (layer "B.Cu") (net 2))
 (segment (start 155.3629 100.8182) (end 156.6129 102.0682) (width 0.2) (layer "B.Cu") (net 2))
 (segment (start 107.5 82.84) (end 107.5 81.6883) (width 0.2) (layer "B.Cu") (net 2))
 (segment (start 106.3468 78.5567) (end 106.3468 80.5351) (width 0.2) (layer "B.Cu") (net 2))
 (segment (start 151.54 91.7453) (end 155.3629 95.5682) (width 0.2) (layer "B.Cu") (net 2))
 (segment (start 125.4085 91.78) (end 151.5429 91.78) (width 0.2) (layer "F.Cu") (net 3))
 (segment (start 118.7349 93.0148) (end 124.1737 93.0148) (width 0.2) (layer "F.Cu") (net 3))
 (segment (start 124.1737 93.0148) (end 125.4085 91.78) (width 0.2) (layer "F.Cu") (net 3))
 (segment (start 151.5429 91.78) (end 155.2947 88.0282) (width 0.2) (layer "F.Cu") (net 3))
 (via (at 118.7349 93.0148) (size 0.6) (drill 0.3) (layers "F.Cu" "B.Cu") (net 3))
 (segment (start 155.2947 81.7147) (end 154.08 80.5) (width 0.2) (layer "B.Cu") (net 3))
 (segment (start 118.7349 98.4726) (end 118.7349 93.0148) (width 0.2) (layer "B.Cu") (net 3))
 (segment (start 160.7743 76.2351) (end 155.2947 81.7147) (width 0.2) (layer "B.Cu") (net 3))
 (segment (start 155.2947 88.0282) (end 155.2947 81.7147) (width 0.2) (layer "B.Cu") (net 3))
 (segment (start 161.79 75.25) (end 160.7743 75.25) (width 0.2) (layer "B.Cu") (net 3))
 (segment (start 160.7743 75.25) (end 160.7743 76.2351) (width 0.2) (layer "B.Cu") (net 3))
 (segment (start 114.035 103.1725) (end 118.7349 98.4726) (width 0.2) (layer "B.Cu") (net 3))
 (segment (start 120.8915 71.92) (end 129.0115 80.04) (width 0.2) (layer "F.Cu") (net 16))
 (segment (start 119 71.92) (end 120.8915 71.92) (width 0.2) (layer "F.Cu") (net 16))
 (segment (start 129.0115 80.04) (end 130.188 80.04) (width 0.2) (layer "F.Cu") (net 16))
 (segment (start 131.22 61.76) (end 131.46 62) (width 0.2) (layer "F.Cu") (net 12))
 (segment (start 119 61.76) (end 131.22 61.76) (width 0.2) (layer "F.Cu") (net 12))
 (segment (start 130.188 68.9568) (end 131.46 67.6848) (width 0.2) (layer "B.Cu") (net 12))
 (segment (start 130.188 69.88) (end 130.188 68.9568) (width 0.2) (layer "B.Cu") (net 12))
 (segment (start 131.46 67.6848) (end 131.46 62) (width 0.2) (layer "B.Cu") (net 12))
 (segment (start 130.188 77.5) (end 127.12 77.5) (width 0.2) (layer "F.Cu") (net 15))
 (segment (start 127.12 77.5) (end 119 69.38) (width 0.2) (layer "F.Cu") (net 15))
 (segment (start 164.5647 95.4353) (end 166 94) (width 0.2) (layer "F.Cu") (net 5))
 (segment (start 151.5329 102.0682) (end 158.1658 95.4353) (width 0.2) (layer "F.Cu") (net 5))
 (segment (start 158.1658 95.4353) (end 164.5647 95.4353) (width 0.2) (layer "F.Cu") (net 5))
 (segment (start 122.045 74.1166) (end 121.1184 73.19) (width 0.2) (layer "F.Cu") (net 7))
 (segment (start 121.1184 73.19) (end 108.73 73.19) (width 0.2) (layer "F.Cu") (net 7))
 (segment (start 121.1184 73.19) (end 122.045 74.1166) (width 0.2) (layer "F.Cu") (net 7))
 (segment (start 122.045 74.1166) (end 121.1184 73.19) (width 0.2) (layer "F.Cu") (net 7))
 (segment (start 108.73 73.19) (end 107.5 71.96) (width 0.2) (layer "F.Cu") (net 7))
 (via (at 122.045 74.1166) (size 0.6) (drill 0.3) (layers "F.Cu" "B.Cu") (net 7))
 (segment (start 131.8654 90.5622) (end 129.8864 88.5832) (width 0.2) (layer "B.Cu") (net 7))
 (segment (start 121.1184 73.19) (end 122.045 74.1166) (width 0.2) (layer "B.Cu") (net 7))
 (segment (start 129.8056 88.5832) (end 122.045 80.8226) (width 0.2) (layer "B.Cu") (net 7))
 (segment (start 131.8654 96.7034) (end 131.8654 90.5622) (width 0.2) (layer "B.Cu") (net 7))
 (segment (start 122.045 74.1166) (end 121.1184 73.19) (width 0.2) (layer "B.Cu") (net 7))
 (segment (start 122.045 80.8226) (end 122.045 74.1166) (width 0.2) (layer "B.Cu") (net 7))
 (segment (start 129.8864 88.5832) (end 129.8056 88.5832) (width 0.2) (layer "B.Cu") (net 7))
 (segment (start 138.062 102.9) (end 131.8654 96.7034) (width 0.2) (layer "B.Cu") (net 7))
 (segment (start 124.939 77.0203) (end 123.767 75.8483) (width 0.2) (layer "F.Cu") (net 8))
 (segment (start 123.767 75.8483) (end 124.939 77.0203) (width 0.2) (layer "F.Cu") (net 8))
 (segment (start 108.8483 75.8483) (end 107.5 74.5) (width 0.2) (layer "F.Cu") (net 8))
 (segment (start 123.767 75.8483) (end 108.8483 75.8483) (width 0.2) (layer "F.Cu") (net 8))
 (segment (start 124.939 77.0203) (end 123.767 75.8483) (width 0.2) (layer "F.Cu") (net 8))
 (via (at 124.939 77.0203) (size 0.6) (drill 0.3) (layers "F.Cu" "B.Cu") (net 8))
 (segment (start 130.451 86.5698) (end 130.3029 86.5698) (width 0.2) (layer "B.Cu") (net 8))
 (segment (start 132.4182 92.1762) (end 132.4182 88.537) (width 0.2) (layer "B.Cu") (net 8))
 (segment (start 130.3029 86.5698) (end 124.939 81.2059) (width 0.2) (layer "B.Cu") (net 8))
 (segment (start 132.4182 88.537) (end 130.451 86.5698) (width 0.2) (layer "B.Cu") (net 8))
 (segment (start 124.939 81.2059) (end 124.939 77.0203) (width 0.2) (layer "B.Cu") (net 8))
 (segment (start 123.767 75.8483) (end 124.939 77.0203) (width 0.2) (layer "B.Cu") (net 8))
 (segment (start 124.939 77.0203) (end 123.767 75.8483) (width 0.2) (layer "B.Cu") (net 8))
 (segment (start 138.062 97.82) (end 132.4182 92.1762) (width 0.2) (layer "B.Cu") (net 8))
 (segment (start 116.85 86.39) (end 107.5 77.04) (width 0.2) (layer "F.Cu") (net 9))
 (segment (start 138.062 87.66) (end 136.792 86.39) (width 0.2) (layer "F.Cu") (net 9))
 (segment (start 136.792 86.39) (end 116.85 86.39) (width 0.2) (layer "F.Cu") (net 9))
 (segment (start 109.0658 78.6058) (end 109.0658 91.4342) (width 0.2) (layer "B.Cu") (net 9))
 (segment (start 107.5 77.04) (end 109.0658 78.6058) (width 0.2) (layer "B.Cu") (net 9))
 (segment (start 109.0658 91.4342) (end 107.5 93) (width 0.2) (layer "B.Cu") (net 9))
 (segment (start 138.062 95.28) (end 137.1388 94.3568) (width 0.2) (layer "F.Cu") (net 25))
 (segment (start 111.3968 94.3568) (end 107.5 90.46) (width 0.2) (layer "F.Cu") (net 25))
 (segment (start 137.1388 94.3568) (end 111.3968 94.3568) (width 0.2) (layer "F.Cu") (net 25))
 (segment (start 106.2839 93.4213) (end 106.2839 89.1361) (width 0.2) (layer "F.Cu") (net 24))
 (segment (start 138.062 100.36) (end 136.792 99.09) (width 0.2) (layer "F.Cu") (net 24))
 (segment (start 111.9526 99.09) (end 106.2839 93.4213) (width 0.2) (layer "F.Cu") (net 24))
 (segment (start 106.2839 89.1361) (end 107.5 87.92) (width 0.2) (layer "F.Cu") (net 24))
 (segment (start 136.792 99.09) (end 111.9526 99.09) (width 0.2) (layer "F.Cu") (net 24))
 (segment (start 120.27 90.3083) (end 117.0217 90.3083) (width 0.2) (layer "B.Cu") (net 6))
 (segment (start 120.27 91.36) (end 120.27 90.3083) (width 0.2) (layer "B.Cu") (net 6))
 (segment (start 117.0217 90.3083) (end 108.955 98.375) (width 0.2) (layer "B.Cu") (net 6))
 (segment (start 108.955 98.375) (end 108.955 103.1725) (width 0.2) (layer "B.Cu") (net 6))
 (segment (start 119.6997 92.4117) (end 119 92.4117) (width 0.2) (layer "B.Cu") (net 23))
 (segment (start 130.188 102.9) (end 119.6997 92.4117) (width 0.2) (layer "B.Cu") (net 23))
 (segment (start 119 91.36) (end 119 92.4117) (width 0.2) (layer "B.Cu") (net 23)))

